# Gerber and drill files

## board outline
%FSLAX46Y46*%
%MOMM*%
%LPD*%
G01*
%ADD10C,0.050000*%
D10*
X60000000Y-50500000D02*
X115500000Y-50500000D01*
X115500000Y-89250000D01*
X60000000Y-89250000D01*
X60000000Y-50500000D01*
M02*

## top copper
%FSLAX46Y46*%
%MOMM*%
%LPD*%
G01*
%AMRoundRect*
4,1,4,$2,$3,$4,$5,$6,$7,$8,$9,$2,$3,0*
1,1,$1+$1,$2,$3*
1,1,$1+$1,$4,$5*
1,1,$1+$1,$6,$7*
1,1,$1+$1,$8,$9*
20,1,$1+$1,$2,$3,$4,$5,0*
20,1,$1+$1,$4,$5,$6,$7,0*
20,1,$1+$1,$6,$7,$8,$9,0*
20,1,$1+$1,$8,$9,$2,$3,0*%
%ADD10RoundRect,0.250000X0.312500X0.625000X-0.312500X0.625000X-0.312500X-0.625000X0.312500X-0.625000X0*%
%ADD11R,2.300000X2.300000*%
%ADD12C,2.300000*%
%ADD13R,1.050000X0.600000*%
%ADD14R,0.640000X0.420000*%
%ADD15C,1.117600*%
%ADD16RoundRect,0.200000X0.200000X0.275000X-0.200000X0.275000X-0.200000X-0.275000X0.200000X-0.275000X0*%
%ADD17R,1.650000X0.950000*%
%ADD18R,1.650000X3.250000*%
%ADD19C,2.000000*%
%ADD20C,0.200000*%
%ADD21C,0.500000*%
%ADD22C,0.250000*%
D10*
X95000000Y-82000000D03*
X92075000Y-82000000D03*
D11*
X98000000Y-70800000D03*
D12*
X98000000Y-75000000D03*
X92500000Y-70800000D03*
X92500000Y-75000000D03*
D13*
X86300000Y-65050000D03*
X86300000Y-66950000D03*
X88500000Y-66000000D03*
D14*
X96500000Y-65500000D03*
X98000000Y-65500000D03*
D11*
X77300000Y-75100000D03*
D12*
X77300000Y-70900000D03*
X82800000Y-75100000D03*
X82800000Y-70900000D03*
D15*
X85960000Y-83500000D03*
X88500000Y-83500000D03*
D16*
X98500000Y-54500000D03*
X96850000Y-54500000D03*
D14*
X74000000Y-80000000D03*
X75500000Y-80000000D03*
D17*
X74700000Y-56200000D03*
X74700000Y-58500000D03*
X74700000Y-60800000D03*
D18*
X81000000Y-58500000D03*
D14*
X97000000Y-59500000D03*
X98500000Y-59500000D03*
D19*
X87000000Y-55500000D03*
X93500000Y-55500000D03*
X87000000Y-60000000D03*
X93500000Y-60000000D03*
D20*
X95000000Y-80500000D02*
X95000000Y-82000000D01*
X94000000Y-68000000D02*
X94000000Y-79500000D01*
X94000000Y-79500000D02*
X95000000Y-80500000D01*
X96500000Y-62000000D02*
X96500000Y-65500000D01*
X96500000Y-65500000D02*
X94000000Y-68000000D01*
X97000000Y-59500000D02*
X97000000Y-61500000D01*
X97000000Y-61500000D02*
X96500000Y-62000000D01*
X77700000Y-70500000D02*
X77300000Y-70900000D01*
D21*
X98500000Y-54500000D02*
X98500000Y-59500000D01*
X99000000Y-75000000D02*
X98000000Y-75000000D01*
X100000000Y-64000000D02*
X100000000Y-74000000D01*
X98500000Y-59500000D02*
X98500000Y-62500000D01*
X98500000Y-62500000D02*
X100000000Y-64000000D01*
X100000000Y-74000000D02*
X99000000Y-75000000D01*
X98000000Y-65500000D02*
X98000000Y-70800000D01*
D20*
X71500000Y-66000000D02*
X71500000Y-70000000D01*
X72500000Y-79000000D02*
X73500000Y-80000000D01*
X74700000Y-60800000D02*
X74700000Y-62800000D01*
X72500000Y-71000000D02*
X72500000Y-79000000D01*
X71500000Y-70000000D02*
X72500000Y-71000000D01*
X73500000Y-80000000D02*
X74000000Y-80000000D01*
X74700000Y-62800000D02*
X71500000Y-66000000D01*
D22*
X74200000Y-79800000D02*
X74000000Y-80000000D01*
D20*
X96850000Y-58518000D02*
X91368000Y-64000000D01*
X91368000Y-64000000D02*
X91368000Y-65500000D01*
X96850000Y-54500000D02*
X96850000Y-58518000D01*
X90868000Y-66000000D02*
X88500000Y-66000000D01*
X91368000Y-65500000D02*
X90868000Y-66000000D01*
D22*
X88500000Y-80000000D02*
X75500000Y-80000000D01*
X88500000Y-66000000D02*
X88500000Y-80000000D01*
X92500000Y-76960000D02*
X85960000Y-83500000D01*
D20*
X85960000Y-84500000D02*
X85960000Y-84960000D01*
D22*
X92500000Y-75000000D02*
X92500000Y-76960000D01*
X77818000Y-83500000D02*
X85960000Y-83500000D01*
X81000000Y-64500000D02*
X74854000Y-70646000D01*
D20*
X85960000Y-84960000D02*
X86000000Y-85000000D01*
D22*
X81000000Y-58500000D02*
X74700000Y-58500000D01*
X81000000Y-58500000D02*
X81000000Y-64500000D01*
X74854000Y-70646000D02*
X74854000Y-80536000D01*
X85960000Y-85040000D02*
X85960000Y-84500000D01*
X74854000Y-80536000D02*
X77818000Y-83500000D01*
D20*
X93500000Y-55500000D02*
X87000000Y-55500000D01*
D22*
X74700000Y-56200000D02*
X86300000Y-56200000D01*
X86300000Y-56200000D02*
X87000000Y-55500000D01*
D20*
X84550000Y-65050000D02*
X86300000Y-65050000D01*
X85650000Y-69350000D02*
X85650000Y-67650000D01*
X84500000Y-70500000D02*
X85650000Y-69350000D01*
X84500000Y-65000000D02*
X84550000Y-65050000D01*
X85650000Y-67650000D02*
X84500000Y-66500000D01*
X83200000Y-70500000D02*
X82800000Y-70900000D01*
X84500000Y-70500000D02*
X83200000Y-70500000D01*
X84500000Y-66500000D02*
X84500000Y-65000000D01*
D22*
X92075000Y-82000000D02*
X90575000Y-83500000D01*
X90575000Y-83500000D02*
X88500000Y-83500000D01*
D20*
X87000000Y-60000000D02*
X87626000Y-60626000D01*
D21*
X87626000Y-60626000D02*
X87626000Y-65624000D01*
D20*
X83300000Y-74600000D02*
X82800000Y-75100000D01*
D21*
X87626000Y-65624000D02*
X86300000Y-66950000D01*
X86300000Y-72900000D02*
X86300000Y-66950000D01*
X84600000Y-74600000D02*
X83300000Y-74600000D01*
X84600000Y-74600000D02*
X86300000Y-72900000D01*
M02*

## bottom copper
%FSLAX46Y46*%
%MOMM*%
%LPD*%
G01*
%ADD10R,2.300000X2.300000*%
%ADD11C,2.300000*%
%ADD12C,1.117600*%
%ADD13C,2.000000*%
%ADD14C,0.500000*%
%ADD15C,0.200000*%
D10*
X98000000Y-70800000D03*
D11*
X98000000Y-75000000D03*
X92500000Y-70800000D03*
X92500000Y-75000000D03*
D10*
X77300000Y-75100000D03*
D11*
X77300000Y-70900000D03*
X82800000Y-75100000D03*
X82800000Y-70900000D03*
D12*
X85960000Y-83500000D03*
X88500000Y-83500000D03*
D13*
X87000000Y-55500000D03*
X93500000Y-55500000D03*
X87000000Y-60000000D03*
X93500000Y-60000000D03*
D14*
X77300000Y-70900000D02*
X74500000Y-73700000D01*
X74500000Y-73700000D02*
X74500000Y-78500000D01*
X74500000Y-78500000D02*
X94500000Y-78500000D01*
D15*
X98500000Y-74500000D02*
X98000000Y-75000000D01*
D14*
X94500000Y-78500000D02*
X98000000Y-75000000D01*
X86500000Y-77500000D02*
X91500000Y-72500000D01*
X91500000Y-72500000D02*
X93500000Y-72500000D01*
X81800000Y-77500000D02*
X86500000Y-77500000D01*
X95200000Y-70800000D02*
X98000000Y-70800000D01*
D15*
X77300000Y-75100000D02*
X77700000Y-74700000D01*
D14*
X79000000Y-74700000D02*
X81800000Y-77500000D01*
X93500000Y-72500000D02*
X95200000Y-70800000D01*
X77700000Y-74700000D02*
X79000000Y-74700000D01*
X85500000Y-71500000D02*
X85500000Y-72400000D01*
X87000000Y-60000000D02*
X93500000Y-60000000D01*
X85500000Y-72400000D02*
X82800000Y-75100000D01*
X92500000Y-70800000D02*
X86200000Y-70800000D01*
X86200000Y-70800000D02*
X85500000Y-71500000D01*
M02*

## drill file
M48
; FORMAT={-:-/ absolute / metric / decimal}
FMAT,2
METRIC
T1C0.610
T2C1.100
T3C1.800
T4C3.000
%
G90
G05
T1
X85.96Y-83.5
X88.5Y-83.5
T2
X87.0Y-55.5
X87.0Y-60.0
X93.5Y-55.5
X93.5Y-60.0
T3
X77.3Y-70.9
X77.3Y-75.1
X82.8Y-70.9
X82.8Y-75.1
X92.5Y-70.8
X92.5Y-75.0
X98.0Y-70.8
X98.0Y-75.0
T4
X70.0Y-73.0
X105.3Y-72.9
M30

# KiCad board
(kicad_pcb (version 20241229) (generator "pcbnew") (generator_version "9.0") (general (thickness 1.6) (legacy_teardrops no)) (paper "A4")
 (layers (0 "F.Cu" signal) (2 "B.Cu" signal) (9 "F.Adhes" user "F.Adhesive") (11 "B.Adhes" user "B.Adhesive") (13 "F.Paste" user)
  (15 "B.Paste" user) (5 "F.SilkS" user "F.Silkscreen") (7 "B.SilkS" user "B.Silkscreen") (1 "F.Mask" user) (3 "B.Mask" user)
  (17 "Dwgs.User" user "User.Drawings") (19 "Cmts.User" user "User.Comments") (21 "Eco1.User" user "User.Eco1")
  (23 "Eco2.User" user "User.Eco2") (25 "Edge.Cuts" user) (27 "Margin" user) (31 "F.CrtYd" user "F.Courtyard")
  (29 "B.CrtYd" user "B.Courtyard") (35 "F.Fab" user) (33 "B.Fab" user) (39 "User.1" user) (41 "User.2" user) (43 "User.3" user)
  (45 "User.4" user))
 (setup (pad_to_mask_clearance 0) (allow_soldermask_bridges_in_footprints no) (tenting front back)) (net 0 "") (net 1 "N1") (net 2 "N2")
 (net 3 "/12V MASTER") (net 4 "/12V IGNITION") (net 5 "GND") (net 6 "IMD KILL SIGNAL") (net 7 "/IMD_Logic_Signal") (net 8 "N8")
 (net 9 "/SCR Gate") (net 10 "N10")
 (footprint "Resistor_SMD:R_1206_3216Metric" (layer "F.Cu") (at 93.5375 82 180)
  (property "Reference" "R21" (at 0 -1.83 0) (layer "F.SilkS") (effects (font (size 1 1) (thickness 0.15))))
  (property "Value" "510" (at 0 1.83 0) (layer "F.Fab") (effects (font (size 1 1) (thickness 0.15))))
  (pad "1" smd roundrect (at -1.4625 0 180) (size 1.125 1.75) (layers "F.Cu" "F.Mask" "F.Paste") (roundrect_rratio 0.222222) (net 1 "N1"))
  (pad "2" smd roundrect (at 1.4625 0 180) (size 1.125 1.75) (layers "F.Cu" "F.Mask" "F.Paste") (roundrect_rratio 0.222222) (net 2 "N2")))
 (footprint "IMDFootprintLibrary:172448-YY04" (layer "F.Cu") (at 98 70.8 90)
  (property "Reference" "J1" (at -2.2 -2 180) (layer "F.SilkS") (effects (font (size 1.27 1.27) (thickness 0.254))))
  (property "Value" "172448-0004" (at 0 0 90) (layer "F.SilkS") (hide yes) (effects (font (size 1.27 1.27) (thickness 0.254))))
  (pad "" np_thru_hole circle (at -2.1 7.3 90) (size 3 3) (drill 3) (layers "*.Cu" "*.Mask"))
  (pad "1" thru_hole rect (at 0 0 90) (size 2.3 2.3) (drill 1.8) (layers "*.Cu" "*.Mask") (remove_unused_layers no) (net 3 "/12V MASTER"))
  (pad "2" thru_hole circle (at -4.2 0 90) (size 2.3 2.3) (drill 1.8) (layers "*.Cu" "*.Mask") (remove_unused_layers no)
   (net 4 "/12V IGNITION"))
  (pad "3" thru_hole circle (at 0 -5.5 90) (size 2.3 2.3) (drill 1.8) (layers "*.Cu" "*.Mask") (remove_unused_layers no) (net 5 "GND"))
  (pad "4" thru_hole circle (at -4.2 -5.5 90) (size 2.3 2.3) (drill 1.8) (layers "*.Cu" "*.Mask") (remove_unused_layers no)
   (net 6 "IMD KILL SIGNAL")))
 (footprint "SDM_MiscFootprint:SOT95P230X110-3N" (layer "F.Cu") (at 87.4 66)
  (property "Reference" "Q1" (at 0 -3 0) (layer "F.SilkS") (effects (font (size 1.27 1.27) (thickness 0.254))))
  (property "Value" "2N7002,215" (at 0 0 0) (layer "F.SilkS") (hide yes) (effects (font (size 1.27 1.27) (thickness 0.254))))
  (pad "1" smd rect (at -1.1 -0.95 90) (size 0.6 1.05) (layers "F.Cu" "F.Mask" "F.Paste") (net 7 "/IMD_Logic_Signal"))
  (pad "2" smd rect (at -1.1 0.95 90) (size 0.6 1.05) (layers "F.Cu" "F.Mask" "F.Paste") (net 5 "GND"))
  (pad "3" smd rect (at 1.1 0 90) (size 0.6 1.05) (layers "F.Cu" "F.Mask" "F.Paste") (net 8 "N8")))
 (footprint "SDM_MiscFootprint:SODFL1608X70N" (layer "F.Cu") (at 97.25 65.5)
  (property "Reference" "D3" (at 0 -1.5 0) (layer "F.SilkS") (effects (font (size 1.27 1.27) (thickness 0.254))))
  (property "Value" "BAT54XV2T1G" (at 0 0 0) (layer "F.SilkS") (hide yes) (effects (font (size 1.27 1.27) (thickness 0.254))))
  (pad "1" smd rect (at -0.75 0 90) (size 0.42 0.64) (layers "F.Cu" "F.Mask" "F.Paste") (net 1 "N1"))
  (pad "2" smd rect (at 0.75 0 90) (size 0.42 0.64) (layers "F.Cu" "F.Mask" "F.Paste") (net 3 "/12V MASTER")))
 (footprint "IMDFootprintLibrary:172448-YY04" (layer "F.Cu") (at 77.3 75.1 -90)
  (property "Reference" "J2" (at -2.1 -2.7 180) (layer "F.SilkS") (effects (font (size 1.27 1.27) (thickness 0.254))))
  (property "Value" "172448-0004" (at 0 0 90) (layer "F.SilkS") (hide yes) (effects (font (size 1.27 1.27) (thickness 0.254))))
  (pad "" np_thru_hole circle (at -2.1 7.3 270) (size 3 3) (drill 3) (layers "*.Cu" "*.Mask"))
  (pad "1" thru_hole rect (at 0 0 270) (size 2.3 2.3) (drill 1.8) (layers "*.Cu" "*.Mask") (remove_unused_layers no) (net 3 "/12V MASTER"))
  (pad "2" thru_hole circle (at -4.2 0 270) (size 2.3 2.3) (drill 1.8) (layers "*.Cu" "*.Mask") (remove_unused_layers no)
   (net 4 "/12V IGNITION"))
  (pad "3" thru_hole circle (at 0 -5.5 270) (size 2.3 2.3) (drill 1.8) (layers "*.Cu" "*.Mask") (remove_unused_layers no) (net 5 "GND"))
  (pad "4" thru_hole circle (at -4.2 -5.5 270) (size 2.3 2.3) (drill 1.8) (layers "*.Cu" "*.Mask") (remove_unused_layers no)
   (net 7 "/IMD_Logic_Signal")))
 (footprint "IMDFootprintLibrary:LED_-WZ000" (layer "F.Cu") (at 85.96 83.5)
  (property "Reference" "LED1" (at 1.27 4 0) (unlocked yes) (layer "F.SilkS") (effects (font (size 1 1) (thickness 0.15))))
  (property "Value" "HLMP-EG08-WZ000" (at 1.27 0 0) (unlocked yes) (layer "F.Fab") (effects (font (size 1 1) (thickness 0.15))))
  (pad "1" thru_hole circle (at 0 0) (size 1.1176 1.1176) (drill 0.6096) (layers "*.Cu" "*.Mask") (remove_unused_layers no)
   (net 6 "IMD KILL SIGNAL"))
  (pad "2" thru_hole circle (at 2.54 0) (size 1.1176 1.1176) (drill 0.6096) (layers "*.Cu" "*.Mask") (remove_unused_layers no) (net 2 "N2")))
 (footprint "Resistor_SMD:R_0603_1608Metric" (layer "F.Cu") (at 97.675 54.5 180)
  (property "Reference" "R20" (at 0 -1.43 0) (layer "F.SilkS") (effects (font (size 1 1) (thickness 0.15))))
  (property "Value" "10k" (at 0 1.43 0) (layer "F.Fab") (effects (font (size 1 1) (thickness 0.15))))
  (pad "1" smd roundrect (at -0.825 0 180) (size 0.8 0.95) (layers "F.Cu" "F.Mask" "F.Paste") (roundrect_rratio 0.25)
   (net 4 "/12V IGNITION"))
  (pad "2" smd roundrect (at 0.825 0 180) (size 0.8 0.95) (layers "F.Cu" "F.Mask" "F.Paste") (roundrect_rratio 0.25) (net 8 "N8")))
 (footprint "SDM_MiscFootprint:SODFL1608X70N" (layer "F.Cu") (at 74.75 80)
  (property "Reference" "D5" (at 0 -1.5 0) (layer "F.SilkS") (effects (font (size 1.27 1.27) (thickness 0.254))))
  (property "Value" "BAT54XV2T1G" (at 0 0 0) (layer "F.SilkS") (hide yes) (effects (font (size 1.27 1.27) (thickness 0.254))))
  (pad "1" smd rect (at -0.75 0 90) (size 0.42 0.64) (layers "F.Cu" "F.Mask" "F.Paste") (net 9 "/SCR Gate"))
  (pad "2" smd rect (at 0.75 0 90) (size 0.42 0.64) (layers "F.Cu" "F.Mask" "F.Paste") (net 8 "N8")))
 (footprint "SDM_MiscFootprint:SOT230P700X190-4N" (layer "F.Cu") (at 77.85 58.5)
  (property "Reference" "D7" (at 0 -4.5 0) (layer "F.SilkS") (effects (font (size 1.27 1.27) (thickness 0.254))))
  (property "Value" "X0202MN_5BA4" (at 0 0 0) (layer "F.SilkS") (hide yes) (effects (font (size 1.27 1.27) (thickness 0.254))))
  (pad "1" smd rect (at -3.15 -2.3 90) (size 0.95 1.65) (layers "F.Cu" "F.Mask" "F.Paste") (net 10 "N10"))
  (pad "2" smd rect (at -3.15 0 90) (size 0.95 1.65) (layers "F.Cu" "F.Mask" "F.Paste") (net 6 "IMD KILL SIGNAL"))
  (pad "3" smd rect (at -3.15 2.3 90) (size 0.95 1.65) (layers "F.Cu" "F.Mask" "F.Paste") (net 9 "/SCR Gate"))
  (pad "4" smd rect (at 3.15 0) (size 1.65 3.25) (layers "F.Cu" "F.Mask" "F.Paste") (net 6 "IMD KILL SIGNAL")))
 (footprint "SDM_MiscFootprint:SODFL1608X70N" (layer "F.Cu") (at 97.75 59.5)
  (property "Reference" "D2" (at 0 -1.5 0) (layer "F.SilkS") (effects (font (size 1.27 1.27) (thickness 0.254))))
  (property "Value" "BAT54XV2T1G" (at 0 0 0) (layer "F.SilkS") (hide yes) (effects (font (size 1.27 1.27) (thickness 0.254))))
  (pad "1" smd rect (at -0.75 0 90) (size 0.42 0.64) (layers "F.Cu" "F.Mask" "F.Paste") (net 1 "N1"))
  (pad "2" smd rect (at 0.75 0 90) (size 0.42 0.64) (layers "F.Cu" "F.Mask" "F.Paste") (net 4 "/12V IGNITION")))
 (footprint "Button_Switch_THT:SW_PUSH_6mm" (layer "F.Cu") (at 87 55.5)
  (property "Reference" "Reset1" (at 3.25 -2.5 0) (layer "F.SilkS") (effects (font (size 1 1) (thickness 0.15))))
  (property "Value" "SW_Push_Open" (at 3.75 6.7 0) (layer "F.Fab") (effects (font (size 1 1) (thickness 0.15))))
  (pad "1" thru_hole circle (at 0 0 90) (size 2 2) (drill 1.1) (layers "*.Cu" "*.Mask") (remove_unused_layers no) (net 10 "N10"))
  (pad "1" thru_hole circle (at 6.5 0 90) (size 2 2) (drill 1.1) (layers "*.Cu" "*.Mask") (remove_unused_layers no) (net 10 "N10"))
  (pad "2" thru_hole circle (at 0 4.5 90) (size 2 2) (drill 1.1) (layers "*.Cu" "*.Mask") (remove_unused_layers no) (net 5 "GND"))
  (pad "2" thru_hole circle (at 6.5 4.5 90) (size 2 2) (drill 1.1) (layers "*.Cu" "*.Mask") (remove_unused_layers no) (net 5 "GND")))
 (gr_rect (start 60 50.5) (end 115.5 89.25) (stroke (width 0.05) (type default)) (fill no) (layer "Edge.Cuts"))
 (segment (start 95 80.5) (end 95 82) (width 0.2) (layer "F.Cu") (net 1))
 (segment (start 94 68) (end 94 79.5) (width 0.2) (layer "F.Cu") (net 1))
 (segment (start 94 79.5) (end 95 80.5) (width 0.2) (layer "F.Cu") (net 1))
 (segment (start 96.5 62) (end 96.5 65.5) (width 0.2) (layer "F.Cu") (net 1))
 (segment (start 96.5 65.5) (end 94 68) (width 0.2) (layer "F.Cu") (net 1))
 (segment (start 97 59.5) (end 97 61.5) (width 0.2) (layer "F.Cu") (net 1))
 (segment (start 97 61.5) (end 96.5 62) (width 0.2) (layer "F.Cu") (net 1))
 (segment (start 77.7 70.5) (end 77.3 70.9) (width 0.2) (layer "F.Cu") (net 4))
 (segment (start 98.5 54.5) (end 98.5 59.5) (width 0.5) (layer "F.Cu") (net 4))
 (segment (start 99 75) (end 98 75) (width 0.5) (layer "F.Cu") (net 4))
 (segment (start 100 64) (end 100 74) (width 0.5) (layer "F.Cu") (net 4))
 (segment (start 98.5 59.5) (end 98.5 62.5) (width 0.5) (layer "F.Cu") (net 4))
 (segment (start 98.5 62.5) (end 100 64) (width 0.5) (layer "F.Cu") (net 4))
 (segment (start 100 74) (end 99 75) (width 0.5) (layer "F.Cu") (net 4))
 (segment (start 77.3 70.9) (end 74.5 73.7) (width 0.5) (layer "B.Cu") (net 4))
 (segment (start 74.5 73.7) (end 74.5 78.5) (width 0.5) (layer "B.Cu") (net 4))
 (segment (start 74.5 78.5) (end 94.5 78.5) (width 0.5) (layer "B.Cu") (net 4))
 (segment (start 98.5 74.5) (end 98 75) (width 0.2) (layer "B.Cu") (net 4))
 (segment (start 94.5 78.5) (end 98 75) (width 0.5) (layer "B.Cu") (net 4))
 (segment (start 98 65.5) (end 98 70.8) (width 0.5) (layer "F.Cu") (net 3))
 (segment (start 86.5 77.5) (end 91.5 72.5) (width 0.5) (layer "B.Cu") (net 3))
 (segment (start 91.5 72.5) (end 93.5 72.5) (width 0.5) (layer "B.Cu") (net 3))
 (segment (start 81.8 77.5) (end 86.5 77.5) (width 0.5) (layer "B.Cu") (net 3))
 (segment (start 95.2 70.8) (end 98 70.8) (width 0.5) (layer "B.Cu") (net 3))
 (segment (start 77.3 75.1) (end 77.7 74.7) (width 0.2) (layer "B.Cu") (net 3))
 (segment (start 79 74.7) (end 81.8 77.5) (width 0.5) (layer "B.Cu") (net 3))
 (segment (start 93.5 72.5) (end 95.2 70.8) (width 0.5) (layer "B.Cu") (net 3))
 (segment (start 77.7 74.7) (end 79 74.7) (width 0.5) (layer "B.Cu") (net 3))
 (segment (start 71.5 66) (end 71.5 70) (width 0.2) (layer "F.Cu") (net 9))
 (segment (start 72.5 79) (end 73.5 80) (width 0.2) (layer "F.Cu") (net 9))
 (segment (start 74.7 60.8) (end 74.7 62.8) (width 0.2) (layer "F.Cu") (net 9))
 (segment (start 72.5 71) (end 72.5 79) (width 0.2) (layer "F.Cu") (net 9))
 (segment (start 71.5 70) (end 72.5 71) (width 0.2) (layer "F.Cu") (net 9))
 (segment (start 73.5 80) (end 74 80) (width 0.2) (layer "F.Cu") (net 9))
 (segment (start 74.7 62.8) (end 71.5 66) (width 0.2) (layer "F.Cu") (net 9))
 (segment (start 74.2 79.8) (end 74 80) (width 0.25) (layer "F.Cu") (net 9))
 (segment (start 96.85 58.518) (end 91.368 64) (width 0.2) (layer "F.Cu") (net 8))
 (segment (start 91.368 64) (end 91.368 65.5) (width 0.2) (layer "F.Cu") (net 8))
 (segment (start 96.85 54.5) (end 96.85 58.518) (width 0.2) (layer "F.Cu") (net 8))
 (segment (start 90.868 66) (end 88.5 66) (width 0.2) (layer "F.Cu") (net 8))
 (segment (start 91.368 65.5) (end 90.868 66) (width 0.2) (layer "F.Cu") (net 8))
 (segment (start 88.5 80) (end 75.5 80) (width 0.25) (layer "F.Cu") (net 8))
 (segment (start 88.5 66) (end 88.5 80) (width 0.25) (layer "F.Cu") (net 8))
 (segment (start 92.5 76.96) (end 85.96 83.5) (width 0.25) (layer "F.Cu") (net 6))
 (segment (start 85.96 84.5) (end 85.96 84.96) (width 0.2) (layer "F.Cu") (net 6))
 (segment (start 92.5 75) (end 92.5 76.96) (width 0.25) (layer "F.Cu") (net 6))
 (segment (start 77.818 83.5) (end 85.96 83.5) (width 0.25) (layer "F.Cu") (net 6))
 (segment (start 81 64.5) (end 74.854 70.646) (width 0.25) (layer "F.Cu") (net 6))
 (segment (start 85.96 84.96) (end 86 85) (width 0.2) (layer "F.Cu") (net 6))
 (segment (start 81 58.5) (end 74.7 58.5) (width 0.25) (layer "F.Cu") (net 6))
 (segment (start 81 58.5) (end 81 64.5) (width 0.25) (layer "F.Cu") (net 6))
 (segment (start 74.854 70.646) (end 74.854 80.536) (width 0.25) (layer "F.Cu") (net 6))
 (segment (start 85.96 85.04) (end 85.96 84.5) (width 0.25) (layer "F.Cu") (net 6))
 (segment (start 74.854 80.536) (end 77.818 83.5) (width 0.25) (layer "F.Cu") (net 6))
 (segment (start 93.5 55.5) (end 87 55.5) (width 0.2) (layer "F.Cu") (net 10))
 (segment (start 74.7 56.2) (end 86.3 56.2) (width 0.25) (layer "F.Cu") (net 10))
 (segment (start 86.3 56.2) (end 87 55.5) (width 0.25) (layer "F.Cu") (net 10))
 (segment (start 84.55 65.05) (end 86.3 65.05) (width 0.2) (layer "F.Cu") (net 7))
 (segment (start 85.65 69.35) (end 85.65 67.65) (width 0.2) (layer "F.Cu") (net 7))
 (segment (start 84.5 70.5) (end 85.65 69.35) (width 0.2) (layer "F.Cu") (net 7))
 (segment (start 84.5 65) (end 84.55 65.05) (width 0.2) (layer "F.Cu") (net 7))
 (segment (start 85.65 67.65) (end 84.5 66.5) (width 0.2) (layer "F.Cu") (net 7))
 (segment (start 83.2 70.5) (end 82.8 70.9) (width 0.2) (layer "F.Cu") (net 7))
 (segment (start 84.5 70.5) (end 83.2 70.5) (width 0.2) (layer "F.Cu") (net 7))
 (segment (start 84.5 66.5) (end 84.5 65) (width 0.2) (layer "F.Cu") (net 7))
 (segment (start 92.075 82) (end 90.575 83.5) (width 0.25) (layer "F.Cu") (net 2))
 (segment (start 90.575 83.5) (end 88.5 83.5) (width 0.25) (layer "F.Cu") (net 2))
 (segment (start 87 60) (end 87.626 60.626) (width 0.2) (layer "F.Cu") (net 5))
 (segment (start 87.626 60.626) (end 87.626 65.624) (width 0.5) (layer "F.Cu") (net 5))
 (segment (start 83.3 74.6) (end 82.8 75.1) (width 0.2) (layer "F.Cu") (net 5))
 (segment (start 87.626 65.624) (end 86.3 66.95) (width 0.5) (layer "F.Cu") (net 5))
 (segment (start 86.3 72.9) (end 86.3 66.95) (width 0.5) (layer "F.Cu") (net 5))
 (segment (start 84.6 74.6) (end 83.3 74.6) (width 0.5) (layer "F.Cu") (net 5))
 (segment (start 84.6 74.6) (end 86.3 72.9) (width 0.5) (layer "F.Cu") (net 5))
 (segment (start 85.5 71.5) (end 85.5 72.4) (width 0.5) (layer "B.Cu") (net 5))
 (segment (start 87 60) (end 93.5 60) (width 0.5) (layer "B.Cu") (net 5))
 (segment (start 85.5 72.4) (end 82.8 75.1) (width 0.5) (layer "B.Cu") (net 5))
 (segment (start 92.5 70.8) (end 86.2 70.8) (width 0.5) (layer "B.Cu") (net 5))
 (segment (start 86.2 70.8) (end 85.5 71.5) (width 0.5) (layer "B.Cu") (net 5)))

